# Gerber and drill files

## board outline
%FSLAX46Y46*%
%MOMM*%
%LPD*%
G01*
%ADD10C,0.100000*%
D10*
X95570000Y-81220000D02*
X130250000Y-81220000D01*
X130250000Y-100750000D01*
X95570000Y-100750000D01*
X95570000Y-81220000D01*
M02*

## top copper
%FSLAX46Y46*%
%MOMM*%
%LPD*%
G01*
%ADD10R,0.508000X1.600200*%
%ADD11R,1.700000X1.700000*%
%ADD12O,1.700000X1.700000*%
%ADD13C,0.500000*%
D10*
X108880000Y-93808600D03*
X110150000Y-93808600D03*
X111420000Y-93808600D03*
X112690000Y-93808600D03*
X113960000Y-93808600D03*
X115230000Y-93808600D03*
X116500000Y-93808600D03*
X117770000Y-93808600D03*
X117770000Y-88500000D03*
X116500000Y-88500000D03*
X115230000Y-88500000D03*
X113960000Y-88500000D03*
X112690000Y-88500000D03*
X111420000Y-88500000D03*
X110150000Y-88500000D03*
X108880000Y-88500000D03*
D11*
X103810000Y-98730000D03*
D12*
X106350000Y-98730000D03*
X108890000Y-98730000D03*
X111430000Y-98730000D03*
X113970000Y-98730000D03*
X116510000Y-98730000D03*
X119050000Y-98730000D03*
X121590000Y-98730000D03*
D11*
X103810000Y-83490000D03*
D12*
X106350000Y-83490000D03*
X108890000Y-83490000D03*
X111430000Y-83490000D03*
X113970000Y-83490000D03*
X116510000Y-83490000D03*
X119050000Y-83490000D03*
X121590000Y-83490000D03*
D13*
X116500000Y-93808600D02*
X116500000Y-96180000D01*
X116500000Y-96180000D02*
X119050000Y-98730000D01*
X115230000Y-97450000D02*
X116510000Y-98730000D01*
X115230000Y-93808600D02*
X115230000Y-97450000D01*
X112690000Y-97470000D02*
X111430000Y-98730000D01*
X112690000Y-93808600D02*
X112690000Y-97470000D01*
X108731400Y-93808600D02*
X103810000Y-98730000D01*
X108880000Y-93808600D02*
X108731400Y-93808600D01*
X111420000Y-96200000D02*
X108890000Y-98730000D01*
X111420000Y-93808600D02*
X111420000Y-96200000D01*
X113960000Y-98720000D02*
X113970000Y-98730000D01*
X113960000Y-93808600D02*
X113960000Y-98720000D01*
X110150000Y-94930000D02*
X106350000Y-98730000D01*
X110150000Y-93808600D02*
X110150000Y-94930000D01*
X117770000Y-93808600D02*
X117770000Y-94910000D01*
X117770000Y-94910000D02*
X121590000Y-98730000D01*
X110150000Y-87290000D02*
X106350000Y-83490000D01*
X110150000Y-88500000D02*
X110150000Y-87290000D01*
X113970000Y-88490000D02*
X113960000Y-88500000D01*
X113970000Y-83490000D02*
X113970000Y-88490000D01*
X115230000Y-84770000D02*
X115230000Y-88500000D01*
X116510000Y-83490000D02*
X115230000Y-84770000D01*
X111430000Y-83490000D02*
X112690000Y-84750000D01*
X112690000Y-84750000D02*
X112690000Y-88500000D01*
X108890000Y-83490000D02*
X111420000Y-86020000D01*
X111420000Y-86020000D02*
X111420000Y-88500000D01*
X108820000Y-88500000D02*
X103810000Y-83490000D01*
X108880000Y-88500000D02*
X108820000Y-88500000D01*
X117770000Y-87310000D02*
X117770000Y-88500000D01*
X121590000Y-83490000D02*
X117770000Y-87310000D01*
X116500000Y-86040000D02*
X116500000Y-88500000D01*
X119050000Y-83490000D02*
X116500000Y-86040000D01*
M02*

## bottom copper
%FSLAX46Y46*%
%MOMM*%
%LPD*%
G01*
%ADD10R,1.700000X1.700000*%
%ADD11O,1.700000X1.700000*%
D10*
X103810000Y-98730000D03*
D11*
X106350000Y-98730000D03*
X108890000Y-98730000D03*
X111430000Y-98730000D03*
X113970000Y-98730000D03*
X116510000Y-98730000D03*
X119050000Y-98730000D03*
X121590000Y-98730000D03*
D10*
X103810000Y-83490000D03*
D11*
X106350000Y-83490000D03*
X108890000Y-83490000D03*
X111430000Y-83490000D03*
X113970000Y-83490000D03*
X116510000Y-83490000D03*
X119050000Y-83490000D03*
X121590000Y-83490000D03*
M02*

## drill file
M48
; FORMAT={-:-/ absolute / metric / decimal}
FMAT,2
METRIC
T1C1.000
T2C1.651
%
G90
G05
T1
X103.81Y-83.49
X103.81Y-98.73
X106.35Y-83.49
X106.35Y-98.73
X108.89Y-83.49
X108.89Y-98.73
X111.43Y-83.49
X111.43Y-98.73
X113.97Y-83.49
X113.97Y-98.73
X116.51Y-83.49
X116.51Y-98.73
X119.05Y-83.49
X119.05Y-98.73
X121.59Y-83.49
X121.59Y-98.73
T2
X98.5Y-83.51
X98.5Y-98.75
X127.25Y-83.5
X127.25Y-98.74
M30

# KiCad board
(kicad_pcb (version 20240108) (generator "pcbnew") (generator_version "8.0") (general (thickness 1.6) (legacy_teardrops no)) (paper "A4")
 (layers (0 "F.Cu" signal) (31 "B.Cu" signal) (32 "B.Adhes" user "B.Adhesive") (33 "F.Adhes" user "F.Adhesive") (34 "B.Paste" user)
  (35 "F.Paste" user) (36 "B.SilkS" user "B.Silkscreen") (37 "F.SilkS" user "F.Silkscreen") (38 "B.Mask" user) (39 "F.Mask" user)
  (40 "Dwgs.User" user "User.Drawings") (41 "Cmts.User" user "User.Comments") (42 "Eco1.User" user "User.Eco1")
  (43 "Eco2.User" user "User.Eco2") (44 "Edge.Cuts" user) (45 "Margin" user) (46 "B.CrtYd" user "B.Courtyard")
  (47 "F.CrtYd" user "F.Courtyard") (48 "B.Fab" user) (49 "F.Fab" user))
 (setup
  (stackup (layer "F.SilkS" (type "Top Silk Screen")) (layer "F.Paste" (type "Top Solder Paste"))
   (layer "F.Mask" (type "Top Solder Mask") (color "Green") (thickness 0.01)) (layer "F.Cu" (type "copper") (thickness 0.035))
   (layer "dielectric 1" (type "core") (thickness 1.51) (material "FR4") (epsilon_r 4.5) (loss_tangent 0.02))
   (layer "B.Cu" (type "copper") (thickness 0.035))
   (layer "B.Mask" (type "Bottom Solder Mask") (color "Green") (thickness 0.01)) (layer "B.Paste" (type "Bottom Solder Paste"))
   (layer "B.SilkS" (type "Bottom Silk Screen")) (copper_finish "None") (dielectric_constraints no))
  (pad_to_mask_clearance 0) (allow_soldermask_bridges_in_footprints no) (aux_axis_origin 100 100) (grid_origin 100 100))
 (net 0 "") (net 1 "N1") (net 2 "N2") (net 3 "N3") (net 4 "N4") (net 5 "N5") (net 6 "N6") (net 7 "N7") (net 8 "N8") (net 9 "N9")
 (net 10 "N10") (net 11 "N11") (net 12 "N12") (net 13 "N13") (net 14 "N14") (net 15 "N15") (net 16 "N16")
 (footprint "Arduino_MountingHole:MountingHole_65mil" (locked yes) (layer "F.Cu") (at 98.5 83.51)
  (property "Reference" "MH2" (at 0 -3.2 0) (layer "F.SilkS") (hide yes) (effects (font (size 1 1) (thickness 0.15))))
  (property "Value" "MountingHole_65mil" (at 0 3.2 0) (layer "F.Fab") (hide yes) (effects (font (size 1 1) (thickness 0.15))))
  (pad "" np_thru_hole circle (at 0 0) (size 1.651 1.651) (drill 1.651) (layers "F&B.Cu" "*.Mask")))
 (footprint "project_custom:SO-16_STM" (layer "F.Cu") (at 113.325 91.1543 90)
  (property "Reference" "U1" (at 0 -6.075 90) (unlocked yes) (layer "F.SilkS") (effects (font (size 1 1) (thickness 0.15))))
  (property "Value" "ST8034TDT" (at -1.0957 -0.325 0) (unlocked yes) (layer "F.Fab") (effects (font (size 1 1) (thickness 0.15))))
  (pad "1" smd rect (at -2.6543 -4.445 90) (size 1.6002 0.508) (layers "F.Cu" "F.Paste" "F.Mask") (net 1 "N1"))
  (pad "2" smd rect (at -2.6543 -3.175 90) (size 1.6002 0.508) (layers "F.Cu" "F.Paste" "F.Mask") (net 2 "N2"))
  (pad "3" smd rect (at -2.6543 -1.905 90) (size 1.6002 0.508) (layers "F.Cu" "F.Paste" "F.Mask") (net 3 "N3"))
  (pad "4" smd rect (at -2.6543 -0.635 90) (size 1.6002 0.508) (layers "F.Cu" "F.Paste" "F.Mask") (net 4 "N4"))
  (pad "5" smd rect (at -2.6543 0.635 90) (size 1.6002 0.508) (layers "F.Cu" "F.Paste" "F.Mask") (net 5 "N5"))
  (pad "6" smd rect (at -2.6543 1.905 90) (size 1.6002 0.508) (layers "F.Cu" "F.Paste" "F.Mask") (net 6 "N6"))
  (pad "7" smd rect (at -2.6543 3.175 90) (size 1.6002 0.508) (layers "F.Cu" "F.Paste" "F.Mask") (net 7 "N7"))
  (pad "8" smd rect (at -2.6543 4.445 90) (size 1.6002 0.508) (layers "F.Cu" "F.Paste" "F.Mask") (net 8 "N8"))
  (pad "9" smd rect (at 2.6543 4.445 90) (size 1.6002 0.508) (layers "F.Cu" "F.Paste" "F.Mask") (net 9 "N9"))
  (pad "10" smd rect (at 2.6543 3.175 90) (size 1.6002 0.508) (layers "F.Cu" "F.Paste" "F.Mask") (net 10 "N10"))
  (pad "11" smd rect (at 2.6543 1.905 90) (size 1.6002 0.508) (layers "F.Cu" "F.Paste" "F.Mask") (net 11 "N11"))
  (pad "12" smd rect (at 2.6543 0.635 90) (size 1.6002 0.508) (layers "F.Cu" "F.Paste" "F.Mask") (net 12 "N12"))
  (pad "13" smd rect (at 2.6543 -0.635 90) (size 1.6002 0.508) (layers "F.Cu" "F.Paste" "F.Mask") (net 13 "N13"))
  (pad "14" smd rect (at 2.6543 -1.905 90) (size 1.6002 0.508) (layers "F.Cu" "F.Paste" "F.Mask") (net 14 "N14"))
  (pad "15" smd rect (at 2.6543 -3.175 90) (size 1.6002 0.508) (layers "F.Cu" "F.Paste" "F.Mask") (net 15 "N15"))
  (pad "16" smd rect (at 2.6543 -4.445 90) (size 1.6002 0.508) (layers "F.Cu" "F.Paste" "F.Mask") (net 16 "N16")))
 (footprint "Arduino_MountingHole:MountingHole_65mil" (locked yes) (layer "F.Cu") (at 127.25 98.74)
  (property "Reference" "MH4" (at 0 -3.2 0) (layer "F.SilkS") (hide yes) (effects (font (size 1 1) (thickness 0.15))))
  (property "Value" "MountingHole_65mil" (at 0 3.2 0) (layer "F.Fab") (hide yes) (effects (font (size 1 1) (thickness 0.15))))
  (pad "" np_thru_hole circle (at 0 0) (size 1.651 1.651) (drill 1.651) (layers "F&B.Cu" "*.Mask")))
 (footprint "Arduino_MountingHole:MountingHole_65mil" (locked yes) (layer "F.Cu") (at 98.5 98.75)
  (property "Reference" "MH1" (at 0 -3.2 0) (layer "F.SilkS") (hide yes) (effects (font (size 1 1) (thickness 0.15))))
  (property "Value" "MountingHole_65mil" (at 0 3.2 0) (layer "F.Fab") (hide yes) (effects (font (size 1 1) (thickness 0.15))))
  (pad "" np_thru_hole circle (at 0 0) (size 1.651 1.651) (drill 1.651) (layers "F&B.Cu" "*.Mask")))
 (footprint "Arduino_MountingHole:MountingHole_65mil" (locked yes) (layer "F.Cu") (at 127.25 83.5)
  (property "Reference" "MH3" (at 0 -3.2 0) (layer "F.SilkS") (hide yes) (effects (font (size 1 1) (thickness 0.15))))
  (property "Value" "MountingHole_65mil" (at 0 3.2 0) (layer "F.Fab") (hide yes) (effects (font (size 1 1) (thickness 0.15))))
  (pad "" np_thru_hole circle (at 0 0) (size 1.651 1.651) (drill 1.651) (layers "F&B.Cu" "*.Mask")))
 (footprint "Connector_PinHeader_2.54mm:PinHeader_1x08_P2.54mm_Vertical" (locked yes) (layer "B.Cu") (at 103.81 98.73 -90)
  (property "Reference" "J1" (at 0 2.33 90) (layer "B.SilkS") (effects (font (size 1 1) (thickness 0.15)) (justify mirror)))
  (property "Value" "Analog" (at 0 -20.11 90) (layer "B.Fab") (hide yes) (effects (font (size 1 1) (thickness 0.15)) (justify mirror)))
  (pad "1" thru_hole rect (at 0 0 270) (size 1.7 1.7) (drill 1) (layers "*.Cu" "*.Mask") (remove_unused_layers no) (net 1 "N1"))
  (pad "2" thru_hole oval (at 0 -2.54 270) (size 1.7 1.7) (drill 1) (layers "*.Cu" "*.Mask") (remove_unused_layers no) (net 2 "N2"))
  (pad "3" thru_hole oval (at 0 -5.08 270) (size 1.7 1.7) (drill 1) (layers "*.Cu" "*.Mask") (remove_unused_layers no) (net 3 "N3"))
  (pad "4" thru_hole oval (at 0 -7.62 270) (size 1.7 1.7) (drill 1) (layers "*.Cu" "*.Mask") (remove_unused_layers no) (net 4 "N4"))
  (pad "5" thru_hole oval (at 0 -10.16 270) (size 1.7 1.7) (drill 1) (layers "*.Cu" "*.Mask") (remove_unused_layers no) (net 5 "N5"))
  (pad "6" thru_hole oval (at 0 -12.7 270) (size 1.7 1.7) (drill 1) (layers "*.Cu" "*.Mask") (remove_unused_layers no) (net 6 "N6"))
  (pad "7" thru_hole oval (at 0 -15.24 270) (size 1.7 1.7) (drill 1) (layers "*.Cu" "*.Mask") (remove_unused_layers no) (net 7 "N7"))
  (pad "8" thru_hole oval (at 0 -17.78 270) (size 1.7 1.7) (drill 1) (layers "*.Cu" "*.Mask") (remove_unused_layers no) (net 8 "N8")))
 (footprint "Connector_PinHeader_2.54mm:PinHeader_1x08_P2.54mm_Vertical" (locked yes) (layer "B.Cu") (at 103.81 83.49 -90)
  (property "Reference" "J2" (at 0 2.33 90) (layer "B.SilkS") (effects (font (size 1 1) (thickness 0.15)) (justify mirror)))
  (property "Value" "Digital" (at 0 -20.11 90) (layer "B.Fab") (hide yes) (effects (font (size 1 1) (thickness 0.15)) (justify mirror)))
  (pad "1" thru_hole rect (at 0 0 270) (size 1.7 1.7) (drill 1) (layers "*.Cu" "*.Mask") (remove_unused_layers no) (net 16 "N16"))
  (pad "2" thru_hole oval (at 0 -2.54 270) (size 1.7 1.7) (drill 1) (layers "*.Cu" "*.Mask") (remove_unused_layers no) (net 15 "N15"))
  (pad "3" thru_hole oval (at 0 -5.08 270) (size 1.7 1.7) (drill 1) (layers "*.Cu" "*.Mask") (remove_unused_layers no) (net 14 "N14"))
  (pad "4" thru_hole oval (at 0 -7.62 270) (size 1.7 1.7) (drill 1) (layers "*.Cu" "*.Mask") (remove_unused_layers no) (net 13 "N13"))
  (pad "5" thru_hole oval (at 0 -10.16 270) (size 1.7 1.7) (drill 1) (layers "*.Cu" "*.Mask") (remove_unused_layers no) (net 12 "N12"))
  (pad "6" thru_hole oval (at 0 -12.7 270) (size 1.7 1.7) (drill 1) (layers "*.Cu" "*.Mask") (remove_unused_layers no) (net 11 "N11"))
  (pad "7" thru_hole oval (at 0 -15.24 270) (size 1.7 1.7) (drill 1) (layers "*.Cu" "*.Mask") (remove_unused_layers no) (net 10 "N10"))
  (pad "8" thru_hole oval (at 0 -17.78 270) (size 1.7 1.7) (drill 1) (layers "*.Cu" "*.Mask") (remove_unused_layers no) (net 9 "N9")))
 (gr_rect (start 95.57 81.22) (end 130.25 100.75) (stroke (width 0.1) (type solid)) (fill none) (layer "Edge.Cuts"))
 (segment (start 116.5 93.8086) (end 116.5 96.18) (width 0.5) (layer "F.Cu") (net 7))
 (segment (start 116.5 96.18) (end 119.05 98.73) (width 0.5) (layer "F.Cu") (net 7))
 (segment (start 115.23 97.45) (end 116.51 98.73) (width 0.5) (layer "F.Cu") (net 6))
 (segment (start 115.23 93.8086) (end 115.23 97.45) (width 0.5) (layer "F.Cu") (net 6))
 (segment (start 112.69 97.47) (end 111.43 98.73) (width 0.5) (layer "F.Cu") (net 4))
 (segment (start 112.69 93.8086) (end 112.69 97.47) (width 0.5) (layer "F.Cu") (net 4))
 (segment (start 108.7314 93.8086) (end 103.81 98.73) (width 0.5) (layer "F.Cu") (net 1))
 (segment (start 108.88 93.8086) (end 108.7314 93.8086) (width 0.5) (layer "F.Cu") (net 1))
 (segment (start 111.42 96.2) (end 108.89 98.73) (width 0.5) (layer "F.Cu") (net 3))
 (segment (start 111.42 93.8086) (end 111.42 96.2) (width 0.5) (layer "F.Cu") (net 3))
 (segment (start 113.96 98.72) (end 113.97 98.73) (width 0.5) (layer "F.Cu") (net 5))
 (segment (start 113.96 93.8086) (end 113.96 98.72) (width 0.5) (layer "F.Cu") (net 5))
 (segment (start 110.15 94.93) (end 106.35 98.73) (width 0.5) (layer "F.Cu") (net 2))
 (segment (start 110.15 93.8086) (end 110.15 94.93) (width 0.5) (layer "F.Cu") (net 2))
 (segment (start 117.77 93.8086) (end 117.77 94.91) (width 0.5) (layer "F.Cu") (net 8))
 (segment (start 117.77 94.91) (end 121.59 98.73) (width 0.5) (layer "F.Cu") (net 8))
 (segment (start 110.15 87.29) (end 106.35 83.49) (width 0.5) (layer "F.Cu") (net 15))
 (segment (start 110.15 88.5) (end 110.15 87.29) (width 0.5) (layer "F.Cu") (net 15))
 (segment (start 113.97 88.49) (end 113.96 88.5) (width 0.5) (layer "F.Cu") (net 12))
 (segment (start 113.97 83.49) (end 113.97 88.49) (width 0.5) (layer "F.Cu") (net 12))
 (segment (start 115.23 84.77) (end 115.23 88.5) (width 0.5) (layer "F.Cu") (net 11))
 (segment (start 116.51 83.49) (end 115.23 84.77) (width 0.5) (layer "F.Cu") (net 11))
 (segment (start 111.43 83.49) (end 112.69 84.75) (width 0.5) (layer "F.Cu") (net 13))
 (segment (start 112.69 84.75) (end 112.69 88.5) (width 0.5) (layer "F.Cu") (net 13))
 (segment (start 108.89 83.49) (end 111.42 86.02) (width 0.5) (layer "F.Cu") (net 14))
 (segment (start 111.42 86.02) (end 111.42 88.5) (width 0.5) (layer "F.Cu") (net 14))
 (segment (start 108.82 88.5) (end 103.81 83.49) (width 0.5) (layer "F.Cu") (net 16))
 (segment (start 108.88 88.5) (end 108.82 88.5) (width 0.5) (layer "F.Cu") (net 16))
 (segment (start 117.77 87.31) (end 117.77 88.5) (width 0.5) (layer "F.Cu") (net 9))
 (segment (start 121.59 83.49) (end 117.77 87.31) (width 0.5) (layer "F.Cu") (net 9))
 (segment (start 116.5 86.04) (end 116.5 88.5) (width 0.5) (layer "F.Cu") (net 10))
 (segment (start 119.05 83.49) (end 116.5 86.04) (width 0.5) (layer "F.Cu") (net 10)))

